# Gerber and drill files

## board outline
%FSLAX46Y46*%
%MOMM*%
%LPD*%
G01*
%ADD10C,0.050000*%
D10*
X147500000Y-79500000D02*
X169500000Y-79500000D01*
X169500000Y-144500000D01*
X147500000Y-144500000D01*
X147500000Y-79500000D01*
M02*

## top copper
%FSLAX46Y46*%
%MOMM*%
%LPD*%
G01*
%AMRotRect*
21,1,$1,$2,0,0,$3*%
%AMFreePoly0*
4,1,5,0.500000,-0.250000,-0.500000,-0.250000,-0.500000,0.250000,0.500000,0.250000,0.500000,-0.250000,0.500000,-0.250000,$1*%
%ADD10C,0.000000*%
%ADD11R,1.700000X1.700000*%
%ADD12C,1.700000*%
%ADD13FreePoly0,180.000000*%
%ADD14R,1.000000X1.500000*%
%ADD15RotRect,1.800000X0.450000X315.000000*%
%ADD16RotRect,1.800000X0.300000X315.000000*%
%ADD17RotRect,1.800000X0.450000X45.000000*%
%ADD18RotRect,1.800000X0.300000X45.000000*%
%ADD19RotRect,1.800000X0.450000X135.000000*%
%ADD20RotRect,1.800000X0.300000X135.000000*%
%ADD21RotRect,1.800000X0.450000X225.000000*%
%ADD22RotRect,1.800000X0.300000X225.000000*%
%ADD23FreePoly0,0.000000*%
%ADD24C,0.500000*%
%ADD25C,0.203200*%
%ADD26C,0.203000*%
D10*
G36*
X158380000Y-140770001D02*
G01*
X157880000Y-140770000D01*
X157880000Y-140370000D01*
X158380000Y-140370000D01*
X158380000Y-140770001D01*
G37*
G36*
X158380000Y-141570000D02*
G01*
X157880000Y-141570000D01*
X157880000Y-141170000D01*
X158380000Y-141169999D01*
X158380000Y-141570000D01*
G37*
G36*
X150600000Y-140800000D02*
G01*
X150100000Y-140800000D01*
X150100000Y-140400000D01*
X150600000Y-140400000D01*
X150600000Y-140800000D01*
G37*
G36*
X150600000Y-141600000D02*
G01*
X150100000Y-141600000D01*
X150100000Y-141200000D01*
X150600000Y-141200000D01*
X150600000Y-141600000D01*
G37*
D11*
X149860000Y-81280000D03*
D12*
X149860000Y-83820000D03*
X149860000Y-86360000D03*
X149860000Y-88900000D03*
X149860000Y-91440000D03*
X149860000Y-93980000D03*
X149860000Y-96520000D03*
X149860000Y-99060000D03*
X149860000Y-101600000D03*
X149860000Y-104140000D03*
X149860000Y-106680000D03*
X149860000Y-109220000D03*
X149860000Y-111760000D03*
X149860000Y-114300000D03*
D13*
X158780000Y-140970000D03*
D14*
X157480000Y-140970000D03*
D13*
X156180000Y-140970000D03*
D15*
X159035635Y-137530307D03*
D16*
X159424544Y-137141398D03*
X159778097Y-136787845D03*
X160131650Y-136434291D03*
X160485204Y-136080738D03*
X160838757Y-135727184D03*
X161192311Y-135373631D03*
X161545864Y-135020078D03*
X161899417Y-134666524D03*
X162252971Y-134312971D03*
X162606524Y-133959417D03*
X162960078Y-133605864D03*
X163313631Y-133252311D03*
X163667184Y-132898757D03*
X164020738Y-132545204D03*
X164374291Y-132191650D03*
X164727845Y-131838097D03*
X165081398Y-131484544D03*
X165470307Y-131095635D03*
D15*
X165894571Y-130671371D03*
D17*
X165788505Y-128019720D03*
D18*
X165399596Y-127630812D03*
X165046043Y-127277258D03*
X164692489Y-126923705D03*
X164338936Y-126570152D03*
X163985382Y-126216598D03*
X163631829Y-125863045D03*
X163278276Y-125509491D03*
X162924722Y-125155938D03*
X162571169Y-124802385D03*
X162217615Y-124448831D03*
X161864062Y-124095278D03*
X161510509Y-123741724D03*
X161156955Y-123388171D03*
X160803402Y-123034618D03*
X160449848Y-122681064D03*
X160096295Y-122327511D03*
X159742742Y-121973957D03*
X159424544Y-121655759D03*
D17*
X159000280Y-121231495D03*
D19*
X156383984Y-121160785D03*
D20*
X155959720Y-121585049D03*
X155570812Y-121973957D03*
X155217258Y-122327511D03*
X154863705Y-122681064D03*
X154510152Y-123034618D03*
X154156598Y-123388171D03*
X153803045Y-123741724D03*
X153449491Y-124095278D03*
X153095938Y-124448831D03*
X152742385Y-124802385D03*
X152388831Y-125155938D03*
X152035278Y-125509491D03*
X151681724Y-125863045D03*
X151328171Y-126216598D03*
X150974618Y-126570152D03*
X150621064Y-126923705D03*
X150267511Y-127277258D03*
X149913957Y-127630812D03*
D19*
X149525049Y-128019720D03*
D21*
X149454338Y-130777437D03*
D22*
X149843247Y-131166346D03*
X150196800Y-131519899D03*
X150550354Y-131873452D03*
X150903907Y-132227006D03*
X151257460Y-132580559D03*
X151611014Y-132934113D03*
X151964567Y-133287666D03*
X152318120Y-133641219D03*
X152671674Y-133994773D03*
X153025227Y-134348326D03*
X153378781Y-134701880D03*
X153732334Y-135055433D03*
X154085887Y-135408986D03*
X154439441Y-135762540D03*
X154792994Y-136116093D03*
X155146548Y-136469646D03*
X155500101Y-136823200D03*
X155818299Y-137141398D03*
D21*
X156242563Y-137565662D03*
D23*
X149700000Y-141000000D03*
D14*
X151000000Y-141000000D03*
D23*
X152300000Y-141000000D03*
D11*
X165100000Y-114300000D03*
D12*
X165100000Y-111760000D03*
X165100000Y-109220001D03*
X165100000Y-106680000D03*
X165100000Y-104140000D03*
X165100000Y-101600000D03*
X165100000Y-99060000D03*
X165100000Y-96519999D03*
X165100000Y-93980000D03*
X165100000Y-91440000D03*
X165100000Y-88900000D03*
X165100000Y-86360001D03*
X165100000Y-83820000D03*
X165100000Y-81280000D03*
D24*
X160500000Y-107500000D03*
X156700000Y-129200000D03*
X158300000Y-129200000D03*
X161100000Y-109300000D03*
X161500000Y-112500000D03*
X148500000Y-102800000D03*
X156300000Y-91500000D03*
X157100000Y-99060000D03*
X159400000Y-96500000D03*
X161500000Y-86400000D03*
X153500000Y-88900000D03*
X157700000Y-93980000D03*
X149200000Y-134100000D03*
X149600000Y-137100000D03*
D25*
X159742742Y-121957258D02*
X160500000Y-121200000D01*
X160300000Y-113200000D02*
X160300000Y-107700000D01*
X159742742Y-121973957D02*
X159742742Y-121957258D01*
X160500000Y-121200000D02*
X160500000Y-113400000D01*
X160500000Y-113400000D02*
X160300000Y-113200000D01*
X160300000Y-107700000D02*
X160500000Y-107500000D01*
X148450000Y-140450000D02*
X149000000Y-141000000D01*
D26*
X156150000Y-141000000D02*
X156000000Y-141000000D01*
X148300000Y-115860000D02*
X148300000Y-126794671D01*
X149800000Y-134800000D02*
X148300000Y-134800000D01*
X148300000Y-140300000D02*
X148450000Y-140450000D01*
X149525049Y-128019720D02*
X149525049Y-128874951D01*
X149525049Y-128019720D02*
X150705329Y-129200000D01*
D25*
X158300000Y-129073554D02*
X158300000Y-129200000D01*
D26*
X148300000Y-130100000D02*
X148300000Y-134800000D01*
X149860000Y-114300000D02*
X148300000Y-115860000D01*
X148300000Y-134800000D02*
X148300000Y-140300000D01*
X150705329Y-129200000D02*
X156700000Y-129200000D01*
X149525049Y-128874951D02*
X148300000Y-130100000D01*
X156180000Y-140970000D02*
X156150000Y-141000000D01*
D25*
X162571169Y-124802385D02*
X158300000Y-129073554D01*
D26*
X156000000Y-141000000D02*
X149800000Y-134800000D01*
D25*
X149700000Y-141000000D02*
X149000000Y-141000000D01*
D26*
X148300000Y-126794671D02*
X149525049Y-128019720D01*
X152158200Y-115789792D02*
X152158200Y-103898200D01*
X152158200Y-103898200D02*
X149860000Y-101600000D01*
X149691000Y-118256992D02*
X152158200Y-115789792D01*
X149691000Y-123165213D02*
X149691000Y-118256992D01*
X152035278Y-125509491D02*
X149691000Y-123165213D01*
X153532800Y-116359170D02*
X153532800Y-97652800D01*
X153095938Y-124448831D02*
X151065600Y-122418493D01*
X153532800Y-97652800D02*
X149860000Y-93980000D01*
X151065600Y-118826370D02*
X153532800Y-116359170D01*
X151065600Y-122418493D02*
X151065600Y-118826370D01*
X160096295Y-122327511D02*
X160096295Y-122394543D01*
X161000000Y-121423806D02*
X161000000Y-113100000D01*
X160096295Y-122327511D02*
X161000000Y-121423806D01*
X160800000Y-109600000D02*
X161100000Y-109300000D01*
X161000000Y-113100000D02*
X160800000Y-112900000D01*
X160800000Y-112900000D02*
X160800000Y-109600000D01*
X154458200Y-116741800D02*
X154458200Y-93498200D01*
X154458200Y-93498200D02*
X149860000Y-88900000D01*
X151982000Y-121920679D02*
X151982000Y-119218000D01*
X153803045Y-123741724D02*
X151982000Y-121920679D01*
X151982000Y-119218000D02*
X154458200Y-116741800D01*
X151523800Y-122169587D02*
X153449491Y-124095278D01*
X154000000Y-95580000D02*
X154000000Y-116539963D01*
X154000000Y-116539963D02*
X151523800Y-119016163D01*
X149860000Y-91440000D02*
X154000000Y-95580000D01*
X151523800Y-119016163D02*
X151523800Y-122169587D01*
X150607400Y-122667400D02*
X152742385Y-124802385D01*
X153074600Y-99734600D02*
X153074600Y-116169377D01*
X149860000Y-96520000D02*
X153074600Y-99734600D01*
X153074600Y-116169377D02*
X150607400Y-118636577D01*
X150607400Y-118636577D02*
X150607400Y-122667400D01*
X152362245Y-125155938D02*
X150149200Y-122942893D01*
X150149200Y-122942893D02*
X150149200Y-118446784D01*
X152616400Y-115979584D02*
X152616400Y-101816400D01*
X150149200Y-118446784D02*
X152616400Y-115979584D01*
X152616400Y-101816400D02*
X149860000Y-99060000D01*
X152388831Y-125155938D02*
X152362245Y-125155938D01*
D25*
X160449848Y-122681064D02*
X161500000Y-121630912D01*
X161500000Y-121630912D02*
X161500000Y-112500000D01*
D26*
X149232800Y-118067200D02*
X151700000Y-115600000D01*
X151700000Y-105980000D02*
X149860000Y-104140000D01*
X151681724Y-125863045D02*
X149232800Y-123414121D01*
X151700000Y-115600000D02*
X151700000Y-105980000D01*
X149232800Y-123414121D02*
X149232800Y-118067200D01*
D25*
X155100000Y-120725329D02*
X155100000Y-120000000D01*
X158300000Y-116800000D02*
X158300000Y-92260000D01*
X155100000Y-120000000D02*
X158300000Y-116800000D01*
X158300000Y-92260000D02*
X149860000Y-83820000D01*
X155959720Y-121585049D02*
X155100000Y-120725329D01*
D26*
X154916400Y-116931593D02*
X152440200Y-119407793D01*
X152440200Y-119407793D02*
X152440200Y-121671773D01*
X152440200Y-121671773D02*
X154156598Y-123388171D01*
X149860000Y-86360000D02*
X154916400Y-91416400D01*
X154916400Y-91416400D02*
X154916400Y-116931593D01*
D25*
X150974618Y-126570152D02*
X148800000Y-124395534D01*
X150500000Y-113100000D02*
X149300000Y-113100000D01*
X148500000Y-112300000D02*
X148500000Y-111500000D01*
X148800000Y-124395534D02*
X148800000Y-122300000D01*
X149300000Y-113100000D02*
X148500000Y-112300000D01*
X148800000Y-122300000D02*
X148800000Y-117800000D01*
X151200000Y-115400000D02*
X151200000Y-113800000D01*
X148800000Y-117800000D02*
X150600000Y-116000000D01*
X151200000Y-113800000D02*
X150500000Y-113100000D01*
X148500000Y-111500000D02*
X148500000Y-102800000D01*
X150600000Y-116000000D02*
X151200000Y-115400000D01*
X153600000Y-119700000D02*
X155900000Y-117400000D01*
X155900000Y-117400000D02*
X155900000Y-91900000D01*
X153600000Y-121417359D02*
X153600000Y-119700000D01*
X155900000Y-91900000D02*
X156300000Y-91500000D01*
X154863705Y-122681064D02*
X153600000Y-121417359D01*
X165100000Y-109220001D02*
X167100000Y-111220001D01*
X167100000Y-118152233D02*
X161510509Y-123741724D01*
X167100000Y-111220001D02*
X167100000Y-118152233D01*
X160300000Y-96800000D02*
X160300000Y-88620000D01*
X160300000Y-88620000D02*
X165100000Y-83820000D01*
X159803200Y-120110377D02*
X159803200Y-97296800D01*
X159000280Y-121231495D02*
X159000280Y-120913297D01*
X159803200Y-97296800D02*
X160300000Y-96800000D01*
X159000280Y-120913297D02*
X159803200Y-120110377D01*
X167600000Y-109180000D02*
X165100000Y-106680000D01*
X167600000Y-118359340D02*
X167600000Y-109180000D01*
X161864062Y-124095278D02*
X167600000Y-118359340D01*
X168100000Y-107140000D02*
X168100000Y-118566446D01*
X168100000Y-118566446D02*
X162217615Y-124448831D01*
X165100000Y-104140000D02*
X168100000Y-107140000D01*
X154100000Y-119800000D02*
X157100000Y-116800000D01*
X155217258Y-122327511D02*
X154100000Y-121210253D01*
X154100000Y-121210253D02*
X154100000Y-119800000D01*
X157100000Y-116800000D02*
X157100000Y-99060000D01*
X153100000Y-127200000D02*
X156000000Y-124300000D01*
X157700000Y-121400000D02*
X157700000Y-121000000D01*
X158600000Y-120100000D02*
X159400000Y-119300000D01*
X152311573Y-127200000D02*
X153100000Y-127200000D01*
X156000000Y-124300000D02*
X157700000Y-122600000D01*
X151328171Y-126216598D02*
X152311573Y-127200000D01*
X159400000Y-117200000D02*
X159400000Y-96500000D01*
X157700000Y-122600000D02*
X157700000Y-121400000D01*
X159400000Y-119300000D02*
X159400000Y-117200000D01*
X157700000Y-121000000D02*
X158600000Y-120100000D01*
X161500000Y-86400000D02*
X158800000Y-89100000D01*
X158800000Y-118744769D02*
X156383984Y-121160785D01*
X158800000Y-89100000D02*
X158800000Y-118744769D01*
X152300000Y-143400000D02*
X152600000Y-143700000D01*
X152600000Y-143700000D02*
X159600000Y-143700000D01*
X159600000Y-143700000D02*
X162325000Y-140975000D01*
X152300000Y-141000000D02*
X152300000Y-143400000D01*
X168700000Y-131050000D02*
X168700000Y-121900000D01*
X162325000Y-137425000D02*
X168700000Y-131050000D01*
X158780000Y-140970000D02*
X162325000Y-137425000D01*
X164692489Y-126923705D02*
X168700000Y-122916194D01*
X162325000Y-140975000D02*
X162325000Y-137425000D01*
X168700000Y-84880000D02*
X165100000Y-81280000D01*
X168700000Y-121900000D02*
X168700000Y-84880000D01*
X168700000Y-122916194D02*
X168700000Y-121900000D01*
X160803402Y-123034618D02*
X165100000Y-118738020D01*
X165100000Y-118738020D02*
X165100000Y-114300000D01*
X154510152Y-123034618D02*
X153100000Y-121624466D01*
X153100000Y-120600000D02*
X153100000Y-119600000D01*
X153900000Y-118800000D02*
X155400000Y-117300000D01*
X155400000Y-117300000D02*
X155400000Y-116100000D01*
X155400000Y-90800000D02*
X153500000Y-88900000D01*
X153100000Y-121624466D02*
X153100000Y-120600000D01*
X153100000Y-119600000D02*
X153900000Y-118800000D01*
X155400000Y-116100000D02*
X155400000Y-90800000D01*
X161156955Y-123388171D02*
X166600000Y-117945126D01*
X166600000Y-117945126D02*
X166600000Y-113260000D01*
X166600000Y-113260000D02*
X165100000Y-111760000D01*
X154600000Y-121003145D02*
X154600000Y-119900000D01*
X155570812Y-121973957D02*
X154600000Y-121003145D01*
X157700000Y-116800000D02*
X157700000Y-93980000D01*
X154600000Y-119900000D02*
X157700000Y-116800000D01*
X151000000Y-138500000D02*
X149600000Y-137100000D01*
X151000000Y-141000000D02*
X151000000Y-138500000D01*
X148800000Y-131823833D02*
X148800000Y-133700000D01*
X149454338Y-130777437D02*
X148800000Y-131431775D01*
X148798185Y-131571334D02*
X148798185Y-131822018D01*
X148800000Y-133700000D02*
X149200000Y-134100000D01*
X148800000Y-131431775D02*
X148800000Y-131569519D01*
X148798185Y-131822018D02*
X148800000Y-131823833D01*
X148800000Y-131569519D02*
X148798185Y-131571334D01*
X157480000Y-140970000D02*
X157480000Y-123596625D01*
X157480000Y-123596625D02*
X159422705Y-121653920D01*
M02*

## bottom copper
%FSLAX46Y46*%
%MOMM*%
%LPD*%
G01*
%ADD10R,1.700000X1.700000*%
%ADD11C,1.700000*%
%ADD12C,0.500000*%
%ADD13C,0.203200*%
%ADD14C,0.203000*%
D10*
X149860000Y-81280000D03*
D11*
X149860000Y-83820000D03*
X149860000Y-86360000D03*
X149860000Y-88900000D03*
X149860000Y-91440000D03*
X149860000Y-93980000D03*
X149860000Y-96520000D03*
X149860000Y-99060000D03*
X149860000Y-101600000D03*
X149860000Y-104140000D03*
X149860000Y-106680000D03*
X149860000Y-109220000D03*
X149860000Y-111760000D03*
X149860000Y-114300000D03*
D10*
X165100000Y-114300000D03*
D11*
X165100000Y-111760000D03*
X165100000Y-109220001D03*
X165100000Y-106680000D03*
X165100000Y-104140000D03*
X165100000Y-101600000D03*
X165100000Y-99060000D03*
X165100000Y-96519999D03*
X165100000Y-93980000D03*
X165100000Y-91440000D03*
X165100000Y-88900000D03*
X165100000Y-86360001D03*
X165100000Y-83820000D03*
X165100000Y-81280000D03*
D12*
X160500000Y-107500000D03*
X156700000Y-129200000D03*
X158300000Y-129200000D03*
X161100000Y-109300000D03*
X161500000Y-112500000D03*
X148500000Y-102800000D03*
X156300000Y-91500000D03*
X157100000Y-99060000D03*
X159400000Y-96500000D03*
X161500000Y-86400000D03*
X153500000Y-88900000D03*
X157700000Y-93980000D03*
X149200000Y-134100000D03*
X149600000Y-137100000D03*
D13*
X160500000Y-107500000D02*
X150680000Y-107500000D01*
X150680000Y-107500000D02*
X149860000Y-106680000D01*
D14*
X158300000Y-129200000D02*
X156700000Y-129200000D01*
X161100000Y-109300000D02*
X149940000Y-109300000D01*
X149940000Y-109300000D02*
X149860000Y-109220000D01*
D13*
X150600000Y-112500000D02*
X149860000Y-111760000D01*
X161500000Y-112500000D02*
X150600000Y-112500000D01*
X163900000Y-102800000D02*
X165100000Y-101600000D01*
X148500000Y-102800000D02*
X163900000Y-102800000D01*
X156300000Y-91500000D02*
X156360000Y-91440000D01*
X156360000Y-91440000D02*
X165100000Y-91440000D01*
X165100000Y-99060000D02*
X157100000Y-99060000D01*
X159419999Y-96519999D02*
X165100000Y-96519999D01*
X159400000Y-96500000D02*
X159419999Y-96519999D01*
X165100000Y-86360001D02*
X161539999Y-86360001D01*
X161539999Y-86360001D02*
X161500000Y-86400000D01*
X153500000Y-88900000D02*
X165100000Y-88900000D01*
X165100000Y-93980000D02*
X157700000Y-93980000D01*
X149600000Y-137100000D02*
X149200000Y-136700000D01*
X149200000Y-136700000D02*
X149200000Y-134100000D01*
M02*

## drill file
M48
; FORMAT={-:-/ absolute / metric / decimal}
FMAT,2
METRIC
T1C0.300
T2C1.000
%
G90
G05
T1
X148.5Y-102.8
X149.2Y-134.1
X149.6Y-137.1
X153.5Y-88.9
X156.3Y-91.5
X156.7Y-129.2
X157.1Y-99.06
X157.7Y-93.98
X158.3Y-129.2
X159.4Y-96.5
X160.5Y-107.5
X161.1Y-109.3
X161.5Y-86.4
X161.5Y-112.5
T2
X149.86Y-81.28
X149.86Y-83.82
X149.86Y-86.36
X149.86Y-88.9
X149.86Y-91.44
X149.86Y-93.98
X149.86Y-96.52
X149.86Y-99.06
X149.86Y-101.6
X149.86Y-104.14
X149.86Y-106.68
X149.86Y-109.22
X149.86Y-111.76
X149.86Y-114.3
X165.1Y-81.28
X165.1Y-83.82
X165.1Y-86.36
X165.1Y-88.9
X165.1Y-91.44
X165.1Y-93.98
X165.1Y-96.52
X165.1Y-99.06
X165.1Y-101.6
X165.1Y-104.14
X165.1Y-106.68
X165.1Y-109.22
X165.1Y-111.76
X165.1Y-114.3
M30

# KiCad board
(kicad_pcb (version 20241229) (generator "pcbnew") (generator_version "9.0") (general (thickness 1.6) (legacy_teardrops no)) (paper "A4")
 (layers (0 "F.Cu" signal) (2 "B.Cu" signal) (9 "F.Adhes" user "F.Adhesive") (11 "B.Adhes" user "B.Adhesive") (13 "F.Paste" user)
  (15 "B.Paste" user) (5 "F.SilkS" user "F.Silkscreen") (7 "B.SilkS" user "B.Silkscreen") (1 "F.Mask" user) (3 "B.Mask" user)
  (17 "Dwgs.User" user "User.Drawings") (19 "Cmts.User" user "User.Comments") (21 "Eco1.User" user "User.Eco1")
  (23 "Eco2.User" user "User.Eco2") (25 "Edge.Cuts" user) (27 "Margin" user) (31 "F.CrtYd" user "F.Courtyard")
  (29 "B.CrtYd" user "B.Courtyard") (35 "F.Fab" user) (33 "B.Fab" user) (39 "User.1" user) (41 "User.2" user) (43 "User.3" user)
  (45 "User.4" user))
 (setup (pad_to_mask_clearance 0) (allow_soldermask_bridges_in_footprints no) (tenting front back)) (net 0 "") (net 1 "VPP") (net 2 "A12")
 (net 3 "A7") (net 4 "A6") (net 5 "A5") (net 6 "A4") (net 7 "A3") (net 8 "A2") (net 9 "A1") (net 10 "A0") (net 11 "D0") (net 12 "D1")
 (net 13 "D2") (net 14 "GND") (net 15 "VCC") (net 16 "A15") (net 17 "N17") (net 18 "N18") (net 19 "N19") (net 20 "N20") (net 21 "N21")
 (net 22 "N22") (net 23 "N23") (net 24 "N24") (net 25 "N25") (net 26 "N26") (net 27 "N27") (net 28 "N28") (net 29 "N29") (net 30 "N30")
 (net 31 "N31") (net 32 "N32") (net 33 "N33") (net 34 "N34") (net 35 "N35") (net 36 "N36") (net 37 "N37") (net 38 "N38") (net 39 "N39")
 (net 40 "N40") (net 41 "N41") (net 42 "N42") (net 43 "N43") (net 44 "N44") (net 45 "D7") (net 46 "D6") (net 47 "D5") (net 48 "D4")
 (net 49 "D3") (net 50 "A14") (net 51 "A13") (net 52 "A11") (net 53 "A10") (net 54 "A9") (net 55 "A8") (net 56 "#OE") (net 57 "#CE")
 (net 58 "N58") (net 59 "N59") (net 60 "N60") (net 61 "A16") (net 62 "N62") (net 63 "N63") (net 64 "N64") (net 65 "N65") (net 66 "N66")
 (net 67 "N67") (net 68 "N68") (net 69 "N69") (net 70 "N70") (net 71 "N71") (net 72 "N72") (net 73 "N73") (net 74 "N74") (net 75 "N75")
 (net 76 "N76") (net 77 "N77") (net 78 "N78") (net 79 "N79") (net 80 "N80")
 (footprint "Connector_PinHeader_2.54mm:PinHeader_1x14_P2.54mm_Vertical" (layer "F.Cu") (at 149.86 81.28)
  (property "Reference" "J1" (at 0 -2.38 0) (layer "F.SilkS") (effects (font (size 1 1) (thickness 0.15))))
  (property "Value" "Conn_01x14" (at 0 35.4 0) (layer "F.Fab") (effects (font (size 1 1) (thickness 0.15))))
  (pad "1" thru_hole rect (at 0 0) (size 1.7 1.7) (drill 1) (layers "*.Cu" "*.Mask") (remove_unused_layers no) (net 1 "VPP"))
  (pad "2" thru_hole circle (at 0 2.54) (size 1.7 1.7) (drill 1) (layers "*.Cu" "*.Mask") (remove_unused_layers no) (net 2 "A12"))
  (pad "3" thru_hole circle (at 0 5.08) (size 1.7 1.7) (drill 1) (layers "*.Cu" "*.Mask") (remove_unused_layers no) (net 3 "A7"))
  (pad "4" thru_hole circle (at 0 7.62) (size 1.7 1.7) (drill 1) (layers "*.Cu" "*.Mask") (remove_unused_layers no) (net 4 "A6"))
  (pad "5" thru_hole circle (at 0 10.16) (size 1.7 1.7) (drill 1) (layers "*.Cu" "*.Mask") (remove_unused_layers no) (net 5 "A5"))
  (pad "6" thru_hole circle (at 0 12.7) (size 1.7 1.7) (drill 1) (layers "*.Cu" "*.Mask") (remove_unused_layers no) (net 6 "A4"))
  (pad "7" thru_hole circle (at 0 15.24) (size 1.7 1.7) (drill 1) (layers "*.Cu" "*.Mask") (remove_unused_layers no) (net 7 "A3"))
  (pad "8" thru_hole circle (at 0 17.78) (size 1.7 1.7) (drill 1) (layers "*.Cu" "*.Mask") (remove_unused_layers no) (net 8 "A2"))
  (pad "9" thru_hole circle (at 0 20.32) (size 1.7 1.7) (drill 1) (layers "*.Cu" "*.Mask") (remove_unused_layers no) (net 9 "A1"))
  (pad "10" thru_hole circle (at 0 22.86) (size 1.7 1.7) (drill 1) (layers "*.Cu" "*.Mask") (remove_unused_layers no) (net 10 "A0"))
  (pad "11" thru_hole circle (at 0 25.4) (size 1.7 1.7) (drill 1) (layers "*.Cu" "*.Mask") (remove_unused_layers no) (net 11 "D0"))
  (pad "12" thru_hole circle (at 0 27.94) (size 1.7 1.7) (drill 1) (layers "*.Cu" "*.Mask") (remove_unused_layers no) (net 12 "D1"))
  (pad "13" thru_hole circle (at 0 30.48) (size 1.7 1.7) (drill 1) (layers "*.Cu" "*.Mask") (remove_unused_layers no) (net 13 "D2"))
  (pad "14" thru_hole circle (at 0 33.02) (size 1.7 1.7) (drill 1) (layers "*.Cu" "*.Mask") (remove_unused_layers no) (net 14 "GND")))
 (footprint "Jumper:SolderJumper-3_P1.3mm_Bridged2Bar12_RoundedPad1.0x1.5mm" (layer "F.Cu") (at 157.48 140.97 180)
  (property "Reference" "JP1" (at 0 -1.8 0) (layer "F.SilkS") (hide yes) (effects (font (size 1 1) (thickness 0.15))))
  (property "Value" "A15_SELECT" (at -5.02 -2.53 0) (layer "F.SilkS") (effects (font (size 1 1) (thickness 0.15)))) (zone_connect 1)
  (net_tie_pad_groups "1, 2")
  (fp_poly (pts (xy -0.9 0.199999) (xy -0.4 0.2) (xy -0.4 0.6) (xy -0.9 0.6)) (stroke (width 0) (type solid)) (fill yes) (layer "F.Cu"))
  (fp_poly (pts (xy -0.9 -0.6) (xy -0.4 -0.6) (xy -0.4 -0.2) (xy -0.9 -0.199999)) (stroke (width 0) (type solid)) (fill yes) (layer "F.Cu"))
  (pad "1" smd custom (at -1.3 0 180) (size 1 0.5) (layers "F.Cu" "F.Mask") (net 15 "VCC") (zone_connect 2) (thermal_bridge_angle 45)
   (options (clearance outline) (anchor rect)) (primitives))
  (pad "2" smd rect (at 0 0 180) (size 1 1.5) (layers "F.Cu" "F.Mask") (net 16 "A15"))
  (pad "3" smd custom (at 1.3 0 180) (size 1 0.5) (layers "F.Cu" "F.Mask") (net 14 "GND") (zone_connect 2) (thermal_bridge_angle 45)
   (options (clearance outline) (anchor rect)) (primitives)))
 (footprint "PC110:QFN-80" (layer "F.Cu") (at 157.48 129.54 -135)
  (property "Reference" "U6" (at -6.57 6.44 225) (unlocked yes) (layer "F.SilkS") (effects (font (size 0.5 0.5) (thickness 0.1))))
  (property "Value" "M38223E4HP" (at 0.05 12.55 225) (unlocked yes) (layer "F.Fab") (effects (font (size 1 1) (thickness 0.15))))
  (pad "1" smd rect (at 4.55 -6.75 315) (size 1.8 0.45) (layers "F.Cu" "F.Mask" "F.Paste") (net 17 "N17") (thermal_bridge_angle 45))
  (pad "2" smd rect (at 4 -6.75 315) (size 1.8 0.3) (layers "F.Cu" "F.Mask" "F.Paste") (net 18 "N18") (thermal_bridge_angle 45))
  (pad "3" smd rect (at 3.5 -6.75 315) (size 1.8 0.3) (layers "F.Cu" "F.Mask" "F.Paste") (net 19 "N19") (thermal_bridge_angle 45))
  (pad "4" smd rect (at 3 -6.75 315) (size 1.8 0.3) (layers "F.Cu" "F.Mask" "F.Paste") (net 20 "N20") (thermal_bridge_angle 45))
  (pad "5" smd rect (at 2.5 -6.75 315) (size 1.8 0.3) (layers "F.Cu" "F.Mask" "F.Paste") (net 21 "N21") (thermal_bridge_angle 45))
  (pad "6" smd rect (at 2 -6.75 315) (size 1.8 0.3) (layers "F.Cu" "F.Mask" "F.Paste") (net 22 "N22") (thermal_bridge_angle 45))
  (pad "7" smd rect (at 1.5 -6.75 315) (size 1.8 0.3) (layers "F.Cu" "F.Mask" "F.Paste") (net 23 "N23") (thermal_bridge_angle 45))
  (pad "8" smd rect (at 1 -6.75 315) (size 1.8 0.3) (layers "F.Cu" "F.Mask" "F.Paste") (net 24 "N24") (thermal_bridge_angle 45))
  (pad "9" smd rect (at 0.5 -6.75 315) (size 1.8 0.3) (layers "F.Cu" "F.Mask" "F.Paste") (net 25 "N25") (thermal_bridge_angle 45))
  (pad "10" smd rect (at 0 -6.75 315) (size 1.8 0.3) (layers "F.Cu" "F.Mask" "F.Paste") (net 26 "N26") (thermal_bridge_angle 45))
  (pad "11" smd rect (at -0.5 -6.75 315) (size 1.8 0.3) (layers "F.Cu" "F.Mask" "F.Paste") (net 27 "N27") (thermal_bridge_angle 45))
  (pad "12" smd rect (at -1 -6.75 315) (size 1.8 0.3) (layers "F.Cu" "F.Mask" "F.Paste") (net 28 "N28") (thermal_bridge_angle 45))
  (pad "13" smd rect (at -1.5 -6.75 315) (size 1.8 0.3) (layers "F.Cu" "F.Mask" "F.Paste") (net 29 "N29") (thermal_bridge_angle 45))
  (pad "14" smd rect (at -2 -6.75 315) (size 1.8 0.3) (layers "F.Cu" "F.Mask" "F.Paste") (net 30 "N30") (thermal_bridge_angle 45))
  (pad "15" smd rect (at -2.5 -6.75 315) (size 1.8 0.3) (layers "F.Cu" "F.Mask" "F.Paste") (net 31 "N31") (thermal_bridge_angle 45))
  (pad "16" smd rect (at -3 -6.75 315) (size 1.8 0.3) (layers "F.Cu" "F.Mask" "F.Paste") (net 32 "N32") (thermal_bridge_angle 45))
  (pad "17" smd rect (at -3.5 -6.75 315) (size 1.8 0.3) (layers "F.Cu" "F.Mask" "F.Paste") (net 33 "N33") (thermal_bridge_angle 45))
  (pad "18" smd rect (at -4 -6.75 315) (size 1.8 0.3) (layers "F.Cu" "F.Mask" "F.Paste") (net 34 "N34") (thermal_bridge_angle 45))
  (pad "19" smd rect (at -4.55 -6.75 315) (size 1.8 0.3) (layers "F.Cu" "F.Mask" "F.Paste") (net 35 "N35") (thermal_bridge_angle 45))
  (pad "20" smd rect (at -5.15 -6.75 315) (size 1.8 0.45) (layers "F.Cu" "F.Mask" "F.Paste") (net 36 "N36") (thermal_bridge_angle 45))
  (pad "21" smd rect (at -6.950001 -4.8 45) (size 1.8 0.45) (layers "F.Cu" "F.Mask" "F.Paste") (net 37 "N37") (thermal_bridge_angle 45))
  (pad "22" smd rect (at -6.95 -4.25 45) (size 1.8 0.3) (layers "F.Cu" "F.Mask" "F.Paste") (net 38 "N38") (thermal_bridge_angle 45))
  (pad "23" smd rect (at -6.950001 -3.75 45) (size 1.8 0.3) (layers "F.Cu" "F.Mask" "F.Paste") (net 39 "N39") (thermal_bridge_angle 45))
  (pad "24" smd rect (at -6.95 -3.25 45) (size 1.8 0.3) (layers "F.Cu" "F.Mask" "F.Paste") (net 15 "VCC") (thermal_bridge_angle 45))
  (pad "25" smd rect (at -6.95 -2.75 45) (size 1.8 0.3) (layers "F.Cu" "F.Mask" "F.Paste") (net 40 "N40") (thermal_bridge_angle 45))
  (pad "26" smd rect (at -6.95 -2.25 45) (size 1.8 0.3) (layers "F.Cu" "F.Mask" "F.Paste") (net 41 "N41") (thermal_bridge_angle 45))
  (pad "27" smd rect (at -6.95 -1.75 45) (size 1.8 0.3) (layers "F.Cu" "F.Mask" "F.Paste") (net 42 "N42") (thermal_bridge_angle 45))
  (pad "28" smd rect (at -6.950001 -1.25 45) (size 1.8 0.3) (layers "F.Cu" "F.Mask" "F.Paste") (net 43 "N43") (thermal_bridge_angle 45))
  (pad "29" smd rect (at -6.95 -0.75 45) (size 1.8 0.3) (layers "F.Cu" "F.Mask" "F.Paste") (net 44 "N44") (thermal_bridge_angle 45))
  (pad "30" smd rect (at -6.95 -0.25 45) (size 1.8 0.3) (layers "F.Cu" "F.Mask" "F.Paste") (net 14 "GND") (thermal_bridge_angle 45))
  (pad "31" smd rect (at -6.95 0.25 45) (size 1.8 0.3) (layers "F.Cu" "F.Mask" "F.Paste") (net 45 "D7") (thermal_bridge_angle 45))
  (pad "32" smd rect (at -6.95 0.75 45) (size 1.8 0.3) (layers "F.Cu" "F.Mask" "F.Paste") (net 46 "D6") (thermal_bridge_angle 45))
  (pad "33" smd rect (at -6.950001 1.25 45) (size 1.8 0.3) (layers "F.Cu" "F.Mask" "F.Paste") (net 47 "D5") (thermal_bridge_angle 45))
  (pad "34" smd rect (at -6.95 1.75 45) (size 1.8 0.3) (layers "F.Cu" "F.Mask" "F.Paste") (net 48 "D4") (thermal_bridge_angle 45))
  (pad "35" smd rect (at -6.95 2.25 45) (size 1.8 0.3) (layers "F.Cu" "F.Mask" "F.Paste") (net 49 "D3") (thermal_bridge_angle 45))
  (pad "36" smd rect (at -6.95 2.75 45) (size 1.8 0.3) (layers "F.Cu" "F.Mask" "F.Paste") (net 13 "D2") (thermal_bridge_angle 45))
  (pad "37" smd rect (at -6.95 3.25 45) (size 1.8 0.3) (layers "F.Cu" "F.Mask" "F.Paste") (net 12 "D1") (thermal_bridge_angle 45))
  (pad "38" smd rect (at -6.950001 3.75 45) (size 1.8 0.3) (layers "F.Cu" "F.Mask" "F.Paste") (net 11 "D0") (thermal_bridge_angle 45))
  (pad "39" smd rect (at -6.950001 4.2 45) (size 1.8 0.3) (layers "F.Cu" "F.Mask" "F.Paste") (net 16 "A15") (thermal_bridge_angle 45))
  (pad "40" smd rect (at -6.950001 4.8 45) (size 1.8 0.45) (layers "F.Cu" "F.Mask" "F.Paste") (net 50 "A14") (thermal_bridge_angle 45))
  (pad "41" smd rect (at -5.149999 6.7 135) (size 1.8 0.45) (layers "F.Cu" "F.Mask" "F.Paste") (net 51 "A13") (thermal_bridge_angle 45))
  (pad "42" smd rect (at -4.549999 6.7 135) (size 1.8 0.3) (layers "F.Cu" "F.Mask" "F.Paste") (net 2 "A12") (thermal_bridge_angle 45))
  (pad "43" smd rect (at -4.000001 6.7 135) (size 1.8 0.3) (layers "F.Cu" "F.Mask" "F.Paste") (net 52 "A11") (thermal_bridge_angle 45))
  (pad "44" smd rect (at -3.5 6.7 135) (size 1.8 0.3) (layers "F.Cu" "F.Mask" "F.Paste") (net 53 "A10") (thermal_bridge_angle 45))
  (pad "45" smd rect (at -3 6.7 135) (size 1.8 0.3) (layers "F.Cu" "F.Mask" "F.Paste") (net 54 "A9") (thermal_bridge_angle 45))
  (pad "46" smd rect (at -2.5 6.699999 135) (size 1.8 0.3) (layers "F.Cu" "F.Mask" "F.Paste") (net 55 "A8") (thermal_bridge_angle 45))
  (pad "47" smd rect (at -2 6.7 135) (size 1.8 0.3) (layers "F.Cu" "F.Mask" "F.Paste") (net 3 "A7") (thermal_bridge_angle 45))
  (pad "48" smd rect (at -1.5 6.7 135) (size 1.8 0.3) (layers "F.Cu" "F.Mask" "F.Paste") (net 4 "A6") (thermal_bridge_angle 45))
  (pad "49" smd rect (at -1 6.7 135) (size 1.8 0.3) (layers "F.Cu" "F.Mask" "F.Paste") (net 5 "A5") (thermal_bridge_angle 45))
  (pad "50" smd rect (at -0.5 6.7 135) (size 1.8 0.3) (layers "F.Cu" "F.Mask" "F.Paste") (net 6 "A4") (thermal_bridge_angle 45))
  (pad "51" smd rect (at 0 6.699999 135) (size 1.8 0.3) (layers "F.Cu" "F.Mask" "F.Paste") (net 7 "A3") (thermal_bridge_angle 45))
  (pad "52" smd rect (at 0.5 6.7 135) (size 1.8 0.3) (layers "F.Cu" "F.Mask" "F.Paste") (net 8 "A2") (thermal_bridge_angle 45))
  (pad "53" smd rect (at 1 6.7 135) (size 1.8 0.3) (layers "F.Cu" "F.Mask" "F.Paste") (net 9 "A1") (thermal_bridge_angle 45))
  (pad "54" smd rect (at 1.5 6.7 135) (size 1.8 0.3) (layers "F.Cu" "F.Mask" "F.Paste") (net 10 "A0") (thermal_bridge_angle 45))
  (pad "55" smd rect (at 2 6.7 135) (size 1.8 0.3) (layers "F.Cu" "F.Mask" "F.Paste") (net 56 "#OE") (thermal_bridge_angle 45))
  (pad "56" smd rect (at 2.5 6.699999 135) (size 1.8 0.3) (layers "F.Cu" "F.Mask" "F.Paste") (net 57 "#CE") (thermal_bridge_angle 45))
  (pad "57" smd rect (at 3 6.7 135) (size 1.8 0.3) (layers "F.Cu" "F.Mask" "F.Paste") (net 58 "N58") (thermal_bridge_angle 45))
  (pad "58" smd rect (at 3.5 6.7 135) (size 1.8 0.3) (layers "F.Cu" "F.Mask" "F.Paste") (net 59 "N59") (thermal_bridge_angle 45))
  (pad "59" smd rect (at 4.000001 6.7 135) (size 1.8 0.3) (layers "F.Cu" "F.Mask" "F.Paste") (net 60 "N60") (thermal_bridge_angle 45))
  (pad "60" smd rect (at 4.549999 6.7 135) (size 1.8 0.45) (layers "F.Cu" "F.Mask" "F.Paste") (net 14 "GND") (thermal_bridge_angle 45))
  (pad "61" smd rect (at 6.55 4.8 225) (size 1.8 0.45) (layers "F.Cu" "F.Mask" "F.Paste") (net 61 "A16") (thermal_bridge_angle 45))
  (pad "62" smd rect (at 6.55 4.25 225) (size 1.8 0.3) (layers "F.Cu" "F.Mask" "F.Paste") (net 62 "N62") (thermal_bridge_angle 45))
  (pad "63" smd rect (at 6.55 3.75 225) (size 1.8 0.3) (layers "F.Cu" "F.Mask" "F.Paste") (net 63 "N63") (thermal_bridge_angle 45))
  (pad "64" smd rect (at 6.549999 3.25 225) (size 1.8 0.3) (layers "F.Cu" "F.Mask" "F.Paste") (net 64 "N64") (thermal_bridge_angle 45))
  (pad "65" smd rect (at 6.55 2.75 225) (size 1.8 0.3) (layers "F.Cu" "F.Mask" "F.Paste") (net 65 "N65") (thermal_bridge_angle 45))
  (pad "66" smd rect (at 6.55 2.25 225) (size 1.8 0.3) (layers "F.Cu" "F.Mask" "F.Paste") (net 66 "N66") (thermal_bridge_angle 45))
  (pad "67" smd rect (at 6.55 1.749999 225) (size 1.8 0.3) (layers "F.Cu" "F.Mask" "F.Paste") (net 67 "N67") (thermal_bridge_angle 45))
  (pad "68" smd rect (at 6.55 1.25 225) (size 1.8 0.3) (layers "F.Cu" "F.Mask" "F.Paste") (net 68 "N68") (thermal_bridge_angle 45))
  (pad "69" smd rect (at 6.55 0.750001 225) (size 1.8 0.3) (layers "F.Cu" "F.Mask" "F.Paste") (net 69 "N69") (thermal_bridge_angle 45))
  (pad "70" smd rect (at 6.55 0.25 225) (size 1.8 0.3) (layers "F.Cu" "F.Mask" "F.Paste") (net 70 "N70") (thermal_bridge_angle 45))
  (pad "71" smd rect (at 6.55 -0.25 225) (size 1.8 0.3) (layers "F.Cu" "F.Mask" "F.Paste") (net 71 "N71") (thermal_bridge_angle 45))
  (pad "72" smd rect (at 6.55 -0.750001 225) (size 1.8 0.3) (layers "F.Cu" "F.Mask" "F.Paste") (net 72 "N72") (thermal_bridge_angle 45))
  (pad "73" smd rect (at 6.55 -1.25 225) (size 1.8 0.3) (layers "F.Cu" "F.Mask" "F.Paste") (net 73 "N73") (thermal_bridge_angle 45))
  (pad "74" smd rect (at 6.55 -1.749999 225) (size 1.8 0.3) (layers "F.Cu" "F.Mask" "F.Paste") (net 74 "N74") (thermal_bridge_angle 45))
  (pad "75" smd rect (at 6.55 -2.25 225) (size 1.8 0.3) (layers "F.Cu" "F.Mask" "F.Paste") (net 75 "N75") (thermal_bridge_angle 45))
  (pad "76" smd rect (at 6.55 -2.75 225) (size 1.8 0.3) (layers "F.Cu" "F.Mask" "F.Paste") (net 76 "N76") (thermal_bridge_angle 45))
  (pad "77" smd rect (at 6.549999 -3.25 225) (size 1.8 0.3) (layers "F.Cu" "F.Mask" "F.Paste") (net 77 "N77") (thermal_bridge_angle 45))
  (pad "78" smd rect (at 6.55 -3.75 225) (size 1.8 0.3) (layers "F.Cu" "F.Mask" "F.Paste") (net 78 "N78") (thermal_bridge_angle 45))
  (pad "79" smd rect (at 6.55 -4.2 225) (size 1.8 0.3) (layers "F.Cu" "F.Mask" "F.Paste") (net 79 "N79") (thermal_bridge_angle 45))
  (pad "80" smd rect (at 6.55 -4.8 225) (size 1.8 0.45) (layers "F.Cu" "F.Mask" "F.Paste") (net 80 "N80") (thermal_bridge_angle 45)))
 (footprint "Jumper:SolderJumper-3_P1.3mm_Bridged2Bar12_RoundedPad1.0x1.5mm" (layer "F.Cu") (at 151 141)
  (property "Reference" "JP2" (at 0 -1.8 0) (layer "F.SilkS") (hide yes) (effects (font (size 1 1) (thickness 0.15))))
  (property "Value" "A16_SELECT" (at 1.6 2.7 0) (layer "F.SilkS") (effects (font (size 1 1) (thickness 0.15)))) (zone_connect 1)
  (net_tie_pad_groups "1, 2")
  (fp_poly (pts (xy -0.9 -0.6) (xy -0.4 -0.6) (xy -0.4 -0.2) (xy -0.9 -0.2)) (stroke (width 0) (type solid)) (fill yes) (layer "F.Cu"))
  (fp_poly (pts (xy -0.9 0.2) (xy -0.4 0.2) (xy -0.4 0.6) (xy -0.9 0.6)) (stroke (width 0) (type solid)) (fill yes) (layer "F.Cu"))
  (pad "1" smd custom (at -1.3 0) (size 1 0.5) (layers "F.Cu" "F.Mask") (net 14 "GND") (zone_connect 2) (thermal_bridge_angle 45)
   (options (clearance outline) (anchor rect)) (primitives))
  (pad "2" smd rect (at 0 0) (size 1 1.5) (layers "F.Cu" "F.Mask") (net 61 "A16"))
  (pad "3" smd custom (at 1.3 0) (size 1 0.5) (layers "F.Cu" "F.Mask") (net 15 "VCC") (zone_connect 2) (thermal_bridge_angle 45)
   (options (clearance outline) (anchor rect)) (primitives)))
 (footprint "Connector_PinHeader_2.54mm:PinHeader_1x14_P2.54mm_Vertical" (layer "F.Cu") (at 165.1 114.3 180)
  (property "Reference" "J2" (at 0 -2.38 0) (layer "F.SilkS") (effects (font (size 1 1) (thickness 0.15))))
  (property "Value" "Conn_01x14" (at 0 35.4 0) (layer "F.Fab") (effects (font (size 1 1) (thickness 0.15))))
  (pad "1" thru_hole rect (at 0 0 180) (size 1.7 1.7) (drill 1) (layers "*.Cu" "*.Mask") (remove_unused_layers no) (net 49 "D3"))
  (pad "2" thru_hole circle (at 0 2.54 180) (size 1.7 1.7) (drill 1) (layers "*.Cu" "*.Mask") (remove_unused_layers no) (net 48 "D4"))
  (pad "3" thru_hole circle (at 0 5.079999 180) (size 1.7 1.7) (drill 1) (layers "*.Cu" "*.Mask") (remove_unused_layers no) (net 47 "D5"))
  (pad "4" thru_hole circle (at 0 7.62 180) (size 1.7 1.7) (drill 1) (layers "*.Cu" "*.Mask") (remove_unused_layers no) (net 46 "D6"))
  (pad "5" thru_hole circle (at 0 10.16 180) (size 1.7 1.7) (drill 1) (layers "*.Cu" "*.Mask") (remove_unused_layers no) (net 45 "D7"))
  (pad "6" thru_hole circle (at 0 12.7 180) (size 1.7 1.7) (drill 1) (layers "*.Cu" "*.Mask") (remove_unused_layers no) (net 57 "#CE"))
  (pad "7" thru_hole circle (at 0 15.24 180) (size 1.7 1.7) (drill 1) (layers "*.Cu" "*.Mask") (remove_unused_layers no) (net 53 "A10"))
  (pad "8" thru_hole circle (at 0 17.780001 180) (size 1.7 1.7) (drill 1) (layers "*.Cu" "*.Mask") (remove_unused_layers no) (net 56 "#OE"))
  (pad "9" thru_hole circle (at 0 20.32 180) (size 1.7 1.7) (drill 1) (layers "*.Cu" "*.Mask") (remove_unused_layers no) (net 52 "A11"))
  (pad "10" thru_hole circle (at 0 22.86 180) (size 1.7 1.7) (drill 1) (layers "*.Cu" "*.Mask") (remove_unused_layers no) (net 54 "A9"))
  (pad "11" thru_hole circle (at 0 25.4 180) (size 1.7 1.7) (drill 1) (layers "*.Cu" "*.Mask") (remove_unused_layers no) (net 55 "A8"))
  (pad "12" thru_hole circle (at 0 27.939999 180) (size 1.7 1.7) (drill 1) (layers "*.Cu" "*.Mask") (remove_unused_layers no) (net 51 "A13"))
  (pad "13" thru_hole circle (at 0 30.48 180) (size 1.7 1.7) (drill 1) (layers "*.Cu" "*.Mask") (remove_unused_layers no) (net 50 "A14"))
  (pad "14" thru_hole circle (at 0 33.02 180) (size 1.7 1.7) (drill 1) (layers "*.Cu" "*.Mask") (remove_unused_layers no) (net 15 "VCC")))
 (gr_rect (start 147.5 79.5) (end 169.5 144.5) (stroke (width 0.05) (type default)) (fill no) (layer "Edge.Cuts"))
 (segment (start 159.742742 121.957258) (end 160.5 121.2) (width 0.2032) (layer "F.Cu") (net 11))
 (segment (start 160.3 113.2) (end 160.3 107.7) (width 0.2032) (layer "F.Cu") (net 11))
 (segment (start 159.742742 121.973957) (end 159.742742 121.957258) (width 0.2032) (layer "F.Cu") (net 11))
 (segment (start 160.5 121.2) (end 160.5 113.4) (width 0.2032) (layer "F.Cu") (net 11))
 (segment (start 160.5 113.4) (end 160.3 113.2) (width 0.2032) (layer "F.Cu") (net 11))
 (segment (start 160.3 107.7) (end 160.5 107.5) (width 0.2032) (layer "F.Cu") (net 11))
 (via (at 160.5 107.5) (size 0.5) (drill 0.3) (layers "F.Cu" "B.Cu") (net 11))
 (segment (start 160.5 107.5) (end 150.68 107.5) (width 0.2032) (layer "B.Cu") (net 11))
 (segment (start 150.68 107.5) (end 149.86 106.68) (width 0.2032) (layer "B.Cu") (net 11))
 (segment (start 148.45 140.45) (end 149 141) (width 0.2032) (layer "F.Cu") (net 14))
 (segment (start 156.15 141) (end 156 141) (width 0.203) (layer "F.Cu") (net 14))
 (segment (start 148.3 115.86) (end 148.3 126.794671) (width 0.203) (layer "F.Cu") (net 14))
 (segment (start 149.8 134.8) (end 148.3 134.8) (width 0.203) (layer "F.Cu") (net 14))
 (segment (start 148.3 140.3) (end 148.45 140.45) (width 0.203) (layer "F.Cu") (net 14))
 (segment (start 149.525049 128.01972) (end 149.525049 128.874951) (width 0.203) (layer "F.Cu") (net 14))
 (segment (start 149.525049 128.01972) (end 150.705329 129.2) (width 0.203) (layer "F.Cu") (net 14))
 (segment (start 158.3 129.073554) (end 158.3 129.2) (width 0.2032) (layer "F.Cu") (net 14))
 (segment (start 148.3 130.1) (end 148.3 134.8) (width 0.203) (layer "F.Cu") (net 14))
 (segment (start 149.86 114.3) (end 148.3 115.86) (width 0.203) (layer "F.Cu") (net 14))
 (segment (start 148.3 134.8) (end 148.3 140.3) (width 0.203) (layer "F.Cu") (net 14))
 (segment (start 150.705329 129.2) (end 156.7 129.2) (width 0.203) (layer "F.Cu") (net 14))
 (segment (start 149.525049 128.874951) (end 148.3 130.1) (width 0.203) (layer "F.Cu") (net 14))
 (segment (start 156.18 140.97) (end 156.15 141) (width 0.203) (layer "F.Cu") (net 14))
 (segment (start 162.571169 124.802385) (end 158.3 129.073554) (width 0.2032) (layer "F.Cu") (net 14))
 (segment (start 156 141) (end 149.8 134.8) (width 0.203) (layer "F.Cu") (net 14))
 (segment (start 149.7 141) (end 149 141) (width 0.2032) (layer "F.Cu") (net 14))
 (segment (start 148.3 126.794671) (end 149.525049 128.01972) (width 0.203) (layer "F.Cu") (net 14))
 (via (at 156.7 129.2) (size 0.5) (drill 0.3) (layers "F.Cu" "B.Cu") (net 14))
 (via (at 158.3 129.2) (size 0.5) (drill 0.3) (layers "F.Cu" "B.Cu") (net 14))
 (segment (start 158.3 129.2) (end 156.7 129.2) (width 0.203) (layer "B.Cu") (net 14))
 (segment (start 152.1582 115.789792) (end 152.1582 103.8982) (width 0.203) (layer "F.Cu") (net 9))
 (segment (start 152.1582 103.8982) (end 149.86 101.6) (width 0.203) (layer "F.Cu") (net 9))
 (segment (start 149.691 118.256992) (end 152.1582 115.789792) (width 0.203) (layer "F.Cu") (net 9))
 (segment (start 149.691 123.165213) (end 149.691 118.256992) (width 0.203) (layer "F.Cu") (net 9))
 (segment (start 152.035278 125.509491) (end 149.691 123.165213) (width 0.203) (layer "F.Cu") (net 9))
 (segment (start 153.5328 116.35917) (end 153.5328 97.6528) (width 0.203) (layer "F.Cu") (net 6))
 (segment (start 153.095938 124.448831) (end 151.0656 122.418493) (width 0.203) (layer "F.Cu") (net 6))
 (segment (start 153.5328 97.6528) (end 149.86 93.98) (width 0.203) (layer "F.Cu") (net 6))
 (segment (start 151.0656 118.82637) (end 153.5328 116.35917) (width 0.203) (layer "F.Cu") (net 6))
 (segment (start 151.0656 122.418493) (end 151.0656 118.82637) (width 0.203) (layer "F.Cu") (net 6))
 (segment (start 160.096295 122.327511) (end 160.096295 122.394543) (width 0.203) (layer "F.Cu") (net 12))
 (segment (start 161 121.423806) (end 161 113.1) (width 0.203) (layer "F.Cu") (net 12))
 (segment (start 160.096295 122.327511) (end 161 121.423806) (width 0.203) (layer "F.Cu") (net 12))
 (segment (start 160.8 109.6) (end 161.1 109.3) (width 0.203) (layer "F.Cu") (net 12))
 (segment (start 161 113.1) (end 160.8 112.9) (width 0.203) (layer "F.Cu") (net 12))
 (segment (start 160.8 112.9) (end 160.8 109.6) (width 0.203) (layer "F.Cu") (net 12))
 (via (at 161.1 109.3) (size 0.5) (drill 0.3) (layers "F.Cu" "B.Cu") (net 12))
 (segment (start 161.1 109.3) (end 149.94 109.3) (width 0.203) (layer "B.Cu") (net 12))
 (segment (start 149.94 109.3) (end 149.86 109.22) (width 0.203) (layer "B.Cu") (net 12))
 (segment (start 154.4582 116.7418) (end 154.4582 93.4982) (width 0.203) (layer "F.Cu") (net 4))
 (segment (start 154.4582 93.4982) (end 149.86 88.9) (width 0.203) (layer "F.Cu") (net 4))
 (segment (start 151.982 121.920679) (end 151.982 119.218) (width 0.203) (layer "F.Cu") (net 4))
 (segment (start 153.803045 123.741724) (end 151.982 121.920679) (width 0.203) (layer "F.Cu") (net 4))
 (segment (start 151.982 119.218) (end 154.4582 116.7418) (width 0.203) (layer "F.Cu") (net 4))
 (segment (start 151.5238 122.169587) (end 153.449491 124.095278) (width 0.203) (layer "F.Cu") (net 5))
 (segment (start 154 95.58) (end 154 116.539963) (width 0.203) (layer "F.Cu") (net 5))
 (segment (start 154 116.539963) (end 151.5238 119.016163) (width 0.203) (layer "F.Cu") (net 5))
 (segment (start 149.86 91.44) (end 154 95.58) (width 0.203) (layer "F.Cu") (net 5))
 (segment (start 151.5238 119.016163) (end 151.5238 122.169587) (width 0.203) (layer "F.Cu") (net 5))
 (segment (start 150.6074 122.6674) (end 152.742385 124.802385) (width 0.203) (layer "F.Cu") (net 7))
 (segment (start 153.0746 99.7346) (end 153.0746 116.169377) (width 0.203) (layer "F.Cu") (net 7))
 (segment (start 149.86 96.52) (end 153.0746 99.7346) (width 0.203) (layer "F.Cu") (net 7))
 (segment (start 153.0746 116.169377) (end 150.6074 118.636577) (width 0.203) (layer "F.Cu") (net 7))
 (segment (start 150.6074 118.636577) (end 150.6074 122.6674) (width 0.203) (layer "F.Cu") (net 7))
 (segment (start 152.362245 125.155938) (end 150.1492 122.942893) (width 0.203) (layer "F.Cu") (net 8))
 (segment (start 150.1492 122.942893) (end 150.1492 118.446784) (width 0.203) (layer "F.Cu") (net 8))
 (segment (start 152.6164 115.979584) (end 152.6164 101.8164) (width 0.203) (layer "F.Cu") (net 8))
 (segment (start 150.1492 118.446784) (end 152.6164 115.979584) (width 0.203) (layer "F.Cu") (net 8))
 (segment (start 152.6164 101.8164) (end 149.86 99.06) (width 0.203) (layer "F.Cu") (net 8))
 (segment (start 152.388831 125.155938) (end 152.362245 125.155938) (width 0.203) (layer "F.Cu") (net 8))
 (segment (start 160.449848 122.681064) (end 161.5 121.630912) (width 0.2032) (layer "F.Cu") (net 13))
 (segment (start 161.5 121.630912) (end 161.5 112.5) (width 0.2032) (layer "F.Cu") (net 13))
 (via (at 161.5 112.5) (size 0.5) (drill 0.3) (layers "F.Cu" "B.Cu") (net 13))
 (segment (start 150.6 112.5) (end 149.86 111.76) (width 0.2032) (layer "B.Cu") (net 13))
 (segment (start 161.5 112.5) (end 150.6 112.5) (width 0.2032) (layer "B.Cu") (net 13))
 (segment (start 149.2328 118.0672) (end 151.7 115.6) (width 0.203) (layer "F.Cu") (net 10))
 (segment (start 151.7 105.98) (end 149.86 104.14) (width 0.203) (layer "F.Cu") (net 10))
 (segment (start 151.681724 125.863045) (end 149.2328 123.414121) (width 0.203) (layer "F.Cu") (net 10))
 (segment (start 151.7 115.6) (end 151.7 105.98) (width 0.203) (layer "F.Cu") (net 10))
 (segment (start 149.2328 123.414121) (end 149.2328 118.0672) (width 0.203) (layer "F.Cu") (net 10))
 (segment (start 155.1 120.725329) (end 155.1 120) (width 0.2032) (layer "F.Cu") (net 2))
 (segment (start 158.3 116.8) (end 158.3 92.26) (width 0.2032) (layer "F.Cu") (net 2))
 (segment (start 155.1 120) (end 158.3 116.8) (width 0.2032) (layer "F.Cu") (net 2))
 (segment (start 158.3 92.26) (end 149.86 83.82) (width 0.2032) (layer "F.Cu") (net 2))
 (segment (start 155.95972 121.585049) (end 155.1 120.725329) (width 0.2032) (layer "F.Cu") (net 2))
 (segment (start 154.9164 116.931593) (end 152.4402 119.407793) (width 0.203) (layer "F.Cu") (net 3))
 (segment (start 152.4402 119.407793) (end 152.4402 121.671773) (width 0.203) (layer "F.Cu") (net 3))
 (segment (start 152.4402 121.671773) (end 154.156598 123.388171) (width 0.203) (layer "F.Cu") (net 3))
 (segment (start 149.86 86.36) (end 154.9164 91.4164) (width 0.203) (layer "F.Cu") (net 3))
 (segment (start 154.9164 91.4164) (end 154.9164 116.931593) (width 0.203) (layer "F.Cu") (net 3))
 (segment (start 150.974618 126.570152) (end 148.8 124.395534) (width 0.2032) (layer "F.Cu") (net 57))
 (segment (start 150.5 113.1) (end 149.3 113.1) (width 0.2032) (layer "F.Cu") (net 57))
 (segment (start 148.5 112.3) (end 148.5 111.5) (width 0.2032) (layer "F.Cu") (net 57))
 (segment (start 148.8 124.395534) (end 148.8 122.3) (width 0.2032) (layer "F.Cu") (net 57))
 (segment (start 149.3 113.1) (end 148.5 112.3) (width 0.2032) (layer "F.Cu") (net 57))
 (segment (start 148.8 122.3) (end 148.8 117.8) (width 0.2032) (layer "F.Cu") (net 57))
 (segment (start 151.2 115.4) (end 151.2 113.8) (width 0.2032) (layer "F.Cu") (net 57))
 (segment (start 148.8 117.8) (end 150.6 116) (width 0.2032) (layer "F.Cu") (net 57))
 (segment (start 151.2 113.8) (end 150.5 113.1) (width 0.2032) (layer "F.Cu") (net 57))
 (segment (start 148.5 111.5) (end 148.5 102.8) (width 0.2032) (layer "F.Cu") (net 57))
 (segment (start 150.6 116) (end 151.2 115.4) (width 0.2032) (layer "F.Cu") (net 57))
 (via (at 148.5 102.8) (size 0.5) (drill 0.3) (layers "F.Cu" "B.Cu") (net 57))
 (segment (start 163.9 102.8) (end 165.1 101.6) (width 0.2032) (layer "B.Cu") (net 57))
 (segment (start 148.5 102.8) (end 163.9 102.8) (width 0.2032) (layer "B.Cu") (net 57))
 (segment (start 153.6 119.7) (end 155.9 117.4) (width 0.2032) (layer "F.Cu") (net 54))
 (segment (start 155.9 117.4) (end 155.9 91.9) (width 0.2032) (layer "F.Cu") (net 54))
 (segment (start 153.6 121.417359) (end 153.6 119.7) (width 0.2032) (layer "F.Cu") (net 54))
 (segment (start 155.9 91.9) (end 156.3 91.5) (width 0.2032) (layer "F.Cu") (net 54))
 (segment (start 154.863705 122.681064) (end 153.6 121.417359) (width 0.2032) (layer "F.Cu") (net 54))
 (via (at 156.3 91.5) (size 0.5) (drill 0.3) (layers "F.Cu" "B.Cu") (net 54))
 (segment (start 156.3 91.5) (end 156.36 91.44) (width 0.2032) (layer "B.Cu") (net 54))
 (segment (start 156.36 91.44) (end 165.1 91.44) (width 0.2032) (layer "B.Cu") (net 54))
 (segment (start 165.1 109.220001) (end 167.1 111.220001) (width 0.2032) (layer "F.Cu") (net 47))
 (segment (start 167.1 118.152233) (end 161.510509 123.741724) (width 0.2032) (layer "F.Cu") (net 47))
 (segment (start 167.1 111.220001) (end 167.1 118.152233) (width 0.2032) (layer "F.Cu") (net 47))
 (segment (start 160.3 96.8) (end 160.3 88.62) (width 0.2032) (layer "F.Cu") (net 50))
 (segment (start 160.3 88.62) (end 165.1 83.82) (width 0.2032) (layer "F.Cu") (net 50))
 (segment (start 159.8032 120.110377) (end 159.8032 97.2968) (width 0.2032) (layer "F.Cu") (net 50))
 (segment (start 159.00028 121.231495) (end 159.00028 120.913297) (width 0.2032) (layer "F.Cu") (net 50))
 (segment (start 159.8032 97.2968) (end 160.3 96.8) (width 0.2032) (layer "F.Cu") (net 50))
 (segment (start 159.00028 120.913297) (end 159.8032 120.110377) (width 0.2032) (layer "F.Cu") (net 50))
 (segment (start 167.6 109.18) (end 165.1 106.68) (width 0.2032) (layer "F.Cu") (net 46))
 (segment (start 167.6 118.35934) (end 167.6 109.18) (width 0.2032) (layer "F.Cu") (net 46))
 (segment (start 161.864062 124.095278) (end 167.6 118.35934) (width 0.2032) (layer "F.Cu") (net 46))
 (segment (start 168.1 107.14) (end 168.1 118.566446) (width 0.2032) (layer "F.Cu") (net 45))
 (segment (start 168.1 118.566446) (end 162.217615 124.448831) (width 0.2032) (layer "F.Cu") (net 45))
 (segment (start 165.1 104.14) (end 168.1 107.14) (width 0.2032) (layer "F.Cu") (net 45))
 (segment (start 154.1 119.8) (end 157.1 116.8) (width 0.2032) (layer "F.Cu") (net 53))
 (segment (start 155.217258 122.327511) (end 154.1 121.210253) (width 0.2032) (layer "F.Cu") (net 53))
 (segment (start 154.1 121.210253) (end 154.1 119.8) (width 0.2032) (layer "F.Cu") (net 53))
 (segment (start 157.1 116.8) (end 157.1 99.06) (width 0.2032) (layer "F.Cu") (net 53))
 (via (at 157.1 99.06) (size 0.5) (drill 0.3) (layers "F.Cu" "B.Cu") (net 53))
 (segment (start 165.1 99.06) (end 157.1 99.06) (width 0.2032) (layer "B.Cu") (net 53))
 (segment (start 153.1 127.2) (end 156 124.3) (width 0.2032) (layer "F.Cu") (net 56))
 (segment (start 157.7 121.4) (end 157.7 121) (width 0.2032) (layer "F.Cu") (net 56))
 (segment (start 158.6 120.1) (end 159.4 119.3) (width 0.2032) (layer "F.Cu") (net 56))
 (segment (start 152.311573 127.2) (end 153.1 127.2) (width 0.2032) (layer "F.Cu") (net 56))
 (segment (start 156 124.3) (end 157.7 122.6) (width 0.2032) (layer "F.Cu") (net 56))
 (segment (start 151.328171 126.216598) (end 152.311573 127.2) (width 0.2032) (layer "F.Cu") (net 56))
 (segment (start 159.4 117.2) (end 159.4 96.5) (width 0.2032) (layer "F.Cu") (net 56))
 (segment (start 157.7 122.6) (end 157.7 121.4) (width 0.2032) (layer "F.Cu") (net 56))
 (segment (start 159.4 119.3) (end 159.4 117.2) (width 0.2032) (layer "F.Cu") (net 56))
 (segment (start 157.7 121) (end 158.6 120.1) (width 0.2032) (layer "F.Cu") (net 56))
 (via (at 159.4 96.5) (size 0.5) (drill 0.3) (layers "F.Cu" "B.Cu") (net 56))
 (segment (start 159.419999 96.519999) (end 165.1 96.519999) (width 0.2032) (layer "B.Cu") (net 56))
 (segment (start 159.4 96.5) (end 159.419999 96.519999) (width 0.2032) (layer "B.Cu") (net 56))
 (segment (start 161.5 86.4) (end 158.8 89.1) (width 0.2032) (layer "F.Cu") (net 51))
 (segment (start 158.8 118.744769) (end 156.383984 121.160785) (width 0.2032) (layer "F.Cu") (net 51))
 (segment (start 158.8 89.1) (end 158.8 118.744769) (width 0.2032) (layer "F.Cu") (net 51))
 (via (at 161.5 86.4) (size 0.5) (drill 0.3) (layers "F.Cu" "B.Cu") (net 51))
 (segment (start 165.1 86.360001) (end 161.539999 86.360001) (width 0.2032) (layer "B.Cu") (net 51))
 (segment (start 161.539999 86.360001) (end 161.5 86.4) (width 0.2032) (layer "B.Cu") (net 51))
 (segment (start 152.3 143.4) (end 152.6 143.7) (width 0.2032) (layer "F.Cu") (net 15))
 (segment (start 152.6 143.7) (end 159.6 143.7) (width 0.2032) (layer "F.Cu") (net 15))
 (segment (start 159.6 143.7) (end 162.325 140.975) (width 0.2032) (layer "F.Cu") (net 15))
 (segment (start 152.3 141) (end 152.3 143.4) (width 0.2032) (layer "F.Cu") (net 15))
 (segment (start 168.7 131.05) (end 168.7 121.9) (width 0.2032) (layer "F.Cu") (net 15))
 (segment (start 162.325 137.425) (end 168.7 131.05) (width 0.2032) (layer "F.Cu") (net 15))
 (segment (start 158.78 140.97) (end 162.325 137.425) (width 0.2032) (layer "F.Cu") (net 15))
 (segment (start 164.692489 126.923705) (end 168.7 122.916194) (width 0.2032) (layer "F.Cu") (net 15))
 (segment (start 162.325 140.975) (end 162.325 137.425) (width 0.2032) (layer "F.Cu") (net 15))
 (segment (start 168.7 84.88) (end 165.1 81.28) (width 0.2032) (layer "F.Cu") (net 15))
 (segment (start 168.7 121.9) (end 168.7 84.88) (width 0.2032) (layer "F.Cu") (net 15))
 (segment (start 168.7 122.916194) (end 168.7 121.9) (width 0.2032) (layer "F.Cu") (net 15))
 (segment (start 160.803402 123.034618) (end 165.1 118.73802) (width 0.2032) (layer "F.Cu") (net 49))
 (segment (start 165.1 118.73802) (end 165.1 114.3) (width 0.2032) (layer "F.Cu") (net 49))
 (segment (start 154.510152 123.034618) (end 153.1 121.624466) (width 0.2032) (layer "F.Cu") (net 55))
 (segment (start 153.1 120.6) (end 153.1 119.6) (width 0.2032) (layer "F.Cu") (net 55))
 (segment (start 153.9 118.8) (end 155.4 117.3) (width 0.2032) (layer "F.Cu") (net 55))
 (segment (start 155.4 117.3) (end 155.4 116.1) (width 0.2032) (layer "F.Cu") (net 55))
 (segment (start 155.4 90.8) (end 153.5 88.9) (width 0.2032) (layer "F.Cu") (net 55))
 (segment (start 153.1 121.624466) (end 153.1 120.6) (width 0.2032) (layer "F.Cu") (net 55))
 (segment (start 153.1 119.6) (end 153.9 118.8) (width 0.2032) (layer "F.Cu") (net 55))
 (segment (start 155.4 116.1) (end 155.4 90.8) (width 0.2032) (layer "F.Cu") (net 55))
 (via (at 153.5 88.9) (size 0.5) (drill 0.3) (layers "F.Cu" "B.Cu") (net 55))
 (segment (start 153.5 88.9) (end 165.1 88.9) (width 0.2032) (layer "B.Cu") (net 55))
 (segment (start 161.156955 123.388171) (end 166.6 117.945126) (width 0.2032) (layer "F.Cu") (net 48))
 (segment (start 166.6 117.945126) (end 166.6 113.26) (width 0.2032) (layer "F.Cu") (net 48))
 (segment (start 166.6 113.26) (end 165.1 111.76) (width 0.2032) (layer "F.Cu") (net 48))
 (segment (start 154.6 121.003145) (end 154.6 119.9) (width 0.2032) (layer "F.Cu") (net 52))
 (segment (start 155.570812 121.973957) (end 154.6 121.003145) (width 0.2032) (layer "F.Cu") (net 52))
 (segment (start 157.7 116.8) (end 157.7 93.98) (width 0.2032) (layer "F.Cu") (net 52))
 (segment (start 154.6 119.9) (end 157.7 116.8) (width 0.2032) (layer "F.Cu") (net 52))
 (via (at 157.7 93.98) (size 0.5) (drill 0.3) (layers "F.Cu" "B.Cu") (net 52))
 (segment (start 165.1 93.98) (end 157.7 93.98) (width 0.2032) (layer "B.Cu") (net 52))
 (segment (start 151 138.5) (end 149.6 137.1) (width 0.2032) (layer "F.Cu") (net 61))
 (segment (start 151 141) (end 151 138.5) (width 0.2032) (layer "F.Cu") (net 61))
 (segment (start 148.8 131.823833) (end 148.8 133.7) (width 0.2032) (layer "F.Cu") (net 61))
 (segment (start 149.454338 130.777437) (end 148.8 131.431775) (width 0.2032) (layer "F.Cu") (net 61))
 (segment (start 148.798185 131.571334) (end 148.798185 131.822018) (width 0.2032) (layer "F.Cu") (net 61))
 (segment (start 148.8 133.7) (end 149.2 134.1) (width 0.2032) (layer "F.Cu") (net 61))
 (segment (start 148.8 131.431775) (end 148.8 131.569519) (width 0.2032) (layer "F.Cu") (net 61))
 (segment (start 148.798185 131.822018) (end 148.8 131.823833) (width 0.2032) (layer "F.Cu") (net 61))
 (segment (start 148.8 131.569519) (end 148.798185 131.571334) (width 0.2032) (layer "F.Cu") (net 61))
 (via (at 149.2 134.1) (size 0.5) (drill 0.3) (layers "F.Cu" "B.Cu") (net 61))
 (via (at 149.6 137.1) (size 0.5) (drill 0.3) (layers "F.Cu" "B.Cu") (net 61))
 (segment (start 149.6 137.1) (end 149.2 136.7) (width 0.2032) (layer "B.Cu") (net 61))
 (segment (start 149.2 136.7) (end 149.2 134.1) (width 0.2032) (layer "B.Cu") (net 61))
 (segment (start 157.48 140.97) (end 157.48 123.596625) (width 0.2032) (layer "F.Cu") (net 16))
 (segment (start 157.48 123.596625) (end 159.422705 121.65392) (width 0.2032) (layer "F.Cu") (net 16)))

